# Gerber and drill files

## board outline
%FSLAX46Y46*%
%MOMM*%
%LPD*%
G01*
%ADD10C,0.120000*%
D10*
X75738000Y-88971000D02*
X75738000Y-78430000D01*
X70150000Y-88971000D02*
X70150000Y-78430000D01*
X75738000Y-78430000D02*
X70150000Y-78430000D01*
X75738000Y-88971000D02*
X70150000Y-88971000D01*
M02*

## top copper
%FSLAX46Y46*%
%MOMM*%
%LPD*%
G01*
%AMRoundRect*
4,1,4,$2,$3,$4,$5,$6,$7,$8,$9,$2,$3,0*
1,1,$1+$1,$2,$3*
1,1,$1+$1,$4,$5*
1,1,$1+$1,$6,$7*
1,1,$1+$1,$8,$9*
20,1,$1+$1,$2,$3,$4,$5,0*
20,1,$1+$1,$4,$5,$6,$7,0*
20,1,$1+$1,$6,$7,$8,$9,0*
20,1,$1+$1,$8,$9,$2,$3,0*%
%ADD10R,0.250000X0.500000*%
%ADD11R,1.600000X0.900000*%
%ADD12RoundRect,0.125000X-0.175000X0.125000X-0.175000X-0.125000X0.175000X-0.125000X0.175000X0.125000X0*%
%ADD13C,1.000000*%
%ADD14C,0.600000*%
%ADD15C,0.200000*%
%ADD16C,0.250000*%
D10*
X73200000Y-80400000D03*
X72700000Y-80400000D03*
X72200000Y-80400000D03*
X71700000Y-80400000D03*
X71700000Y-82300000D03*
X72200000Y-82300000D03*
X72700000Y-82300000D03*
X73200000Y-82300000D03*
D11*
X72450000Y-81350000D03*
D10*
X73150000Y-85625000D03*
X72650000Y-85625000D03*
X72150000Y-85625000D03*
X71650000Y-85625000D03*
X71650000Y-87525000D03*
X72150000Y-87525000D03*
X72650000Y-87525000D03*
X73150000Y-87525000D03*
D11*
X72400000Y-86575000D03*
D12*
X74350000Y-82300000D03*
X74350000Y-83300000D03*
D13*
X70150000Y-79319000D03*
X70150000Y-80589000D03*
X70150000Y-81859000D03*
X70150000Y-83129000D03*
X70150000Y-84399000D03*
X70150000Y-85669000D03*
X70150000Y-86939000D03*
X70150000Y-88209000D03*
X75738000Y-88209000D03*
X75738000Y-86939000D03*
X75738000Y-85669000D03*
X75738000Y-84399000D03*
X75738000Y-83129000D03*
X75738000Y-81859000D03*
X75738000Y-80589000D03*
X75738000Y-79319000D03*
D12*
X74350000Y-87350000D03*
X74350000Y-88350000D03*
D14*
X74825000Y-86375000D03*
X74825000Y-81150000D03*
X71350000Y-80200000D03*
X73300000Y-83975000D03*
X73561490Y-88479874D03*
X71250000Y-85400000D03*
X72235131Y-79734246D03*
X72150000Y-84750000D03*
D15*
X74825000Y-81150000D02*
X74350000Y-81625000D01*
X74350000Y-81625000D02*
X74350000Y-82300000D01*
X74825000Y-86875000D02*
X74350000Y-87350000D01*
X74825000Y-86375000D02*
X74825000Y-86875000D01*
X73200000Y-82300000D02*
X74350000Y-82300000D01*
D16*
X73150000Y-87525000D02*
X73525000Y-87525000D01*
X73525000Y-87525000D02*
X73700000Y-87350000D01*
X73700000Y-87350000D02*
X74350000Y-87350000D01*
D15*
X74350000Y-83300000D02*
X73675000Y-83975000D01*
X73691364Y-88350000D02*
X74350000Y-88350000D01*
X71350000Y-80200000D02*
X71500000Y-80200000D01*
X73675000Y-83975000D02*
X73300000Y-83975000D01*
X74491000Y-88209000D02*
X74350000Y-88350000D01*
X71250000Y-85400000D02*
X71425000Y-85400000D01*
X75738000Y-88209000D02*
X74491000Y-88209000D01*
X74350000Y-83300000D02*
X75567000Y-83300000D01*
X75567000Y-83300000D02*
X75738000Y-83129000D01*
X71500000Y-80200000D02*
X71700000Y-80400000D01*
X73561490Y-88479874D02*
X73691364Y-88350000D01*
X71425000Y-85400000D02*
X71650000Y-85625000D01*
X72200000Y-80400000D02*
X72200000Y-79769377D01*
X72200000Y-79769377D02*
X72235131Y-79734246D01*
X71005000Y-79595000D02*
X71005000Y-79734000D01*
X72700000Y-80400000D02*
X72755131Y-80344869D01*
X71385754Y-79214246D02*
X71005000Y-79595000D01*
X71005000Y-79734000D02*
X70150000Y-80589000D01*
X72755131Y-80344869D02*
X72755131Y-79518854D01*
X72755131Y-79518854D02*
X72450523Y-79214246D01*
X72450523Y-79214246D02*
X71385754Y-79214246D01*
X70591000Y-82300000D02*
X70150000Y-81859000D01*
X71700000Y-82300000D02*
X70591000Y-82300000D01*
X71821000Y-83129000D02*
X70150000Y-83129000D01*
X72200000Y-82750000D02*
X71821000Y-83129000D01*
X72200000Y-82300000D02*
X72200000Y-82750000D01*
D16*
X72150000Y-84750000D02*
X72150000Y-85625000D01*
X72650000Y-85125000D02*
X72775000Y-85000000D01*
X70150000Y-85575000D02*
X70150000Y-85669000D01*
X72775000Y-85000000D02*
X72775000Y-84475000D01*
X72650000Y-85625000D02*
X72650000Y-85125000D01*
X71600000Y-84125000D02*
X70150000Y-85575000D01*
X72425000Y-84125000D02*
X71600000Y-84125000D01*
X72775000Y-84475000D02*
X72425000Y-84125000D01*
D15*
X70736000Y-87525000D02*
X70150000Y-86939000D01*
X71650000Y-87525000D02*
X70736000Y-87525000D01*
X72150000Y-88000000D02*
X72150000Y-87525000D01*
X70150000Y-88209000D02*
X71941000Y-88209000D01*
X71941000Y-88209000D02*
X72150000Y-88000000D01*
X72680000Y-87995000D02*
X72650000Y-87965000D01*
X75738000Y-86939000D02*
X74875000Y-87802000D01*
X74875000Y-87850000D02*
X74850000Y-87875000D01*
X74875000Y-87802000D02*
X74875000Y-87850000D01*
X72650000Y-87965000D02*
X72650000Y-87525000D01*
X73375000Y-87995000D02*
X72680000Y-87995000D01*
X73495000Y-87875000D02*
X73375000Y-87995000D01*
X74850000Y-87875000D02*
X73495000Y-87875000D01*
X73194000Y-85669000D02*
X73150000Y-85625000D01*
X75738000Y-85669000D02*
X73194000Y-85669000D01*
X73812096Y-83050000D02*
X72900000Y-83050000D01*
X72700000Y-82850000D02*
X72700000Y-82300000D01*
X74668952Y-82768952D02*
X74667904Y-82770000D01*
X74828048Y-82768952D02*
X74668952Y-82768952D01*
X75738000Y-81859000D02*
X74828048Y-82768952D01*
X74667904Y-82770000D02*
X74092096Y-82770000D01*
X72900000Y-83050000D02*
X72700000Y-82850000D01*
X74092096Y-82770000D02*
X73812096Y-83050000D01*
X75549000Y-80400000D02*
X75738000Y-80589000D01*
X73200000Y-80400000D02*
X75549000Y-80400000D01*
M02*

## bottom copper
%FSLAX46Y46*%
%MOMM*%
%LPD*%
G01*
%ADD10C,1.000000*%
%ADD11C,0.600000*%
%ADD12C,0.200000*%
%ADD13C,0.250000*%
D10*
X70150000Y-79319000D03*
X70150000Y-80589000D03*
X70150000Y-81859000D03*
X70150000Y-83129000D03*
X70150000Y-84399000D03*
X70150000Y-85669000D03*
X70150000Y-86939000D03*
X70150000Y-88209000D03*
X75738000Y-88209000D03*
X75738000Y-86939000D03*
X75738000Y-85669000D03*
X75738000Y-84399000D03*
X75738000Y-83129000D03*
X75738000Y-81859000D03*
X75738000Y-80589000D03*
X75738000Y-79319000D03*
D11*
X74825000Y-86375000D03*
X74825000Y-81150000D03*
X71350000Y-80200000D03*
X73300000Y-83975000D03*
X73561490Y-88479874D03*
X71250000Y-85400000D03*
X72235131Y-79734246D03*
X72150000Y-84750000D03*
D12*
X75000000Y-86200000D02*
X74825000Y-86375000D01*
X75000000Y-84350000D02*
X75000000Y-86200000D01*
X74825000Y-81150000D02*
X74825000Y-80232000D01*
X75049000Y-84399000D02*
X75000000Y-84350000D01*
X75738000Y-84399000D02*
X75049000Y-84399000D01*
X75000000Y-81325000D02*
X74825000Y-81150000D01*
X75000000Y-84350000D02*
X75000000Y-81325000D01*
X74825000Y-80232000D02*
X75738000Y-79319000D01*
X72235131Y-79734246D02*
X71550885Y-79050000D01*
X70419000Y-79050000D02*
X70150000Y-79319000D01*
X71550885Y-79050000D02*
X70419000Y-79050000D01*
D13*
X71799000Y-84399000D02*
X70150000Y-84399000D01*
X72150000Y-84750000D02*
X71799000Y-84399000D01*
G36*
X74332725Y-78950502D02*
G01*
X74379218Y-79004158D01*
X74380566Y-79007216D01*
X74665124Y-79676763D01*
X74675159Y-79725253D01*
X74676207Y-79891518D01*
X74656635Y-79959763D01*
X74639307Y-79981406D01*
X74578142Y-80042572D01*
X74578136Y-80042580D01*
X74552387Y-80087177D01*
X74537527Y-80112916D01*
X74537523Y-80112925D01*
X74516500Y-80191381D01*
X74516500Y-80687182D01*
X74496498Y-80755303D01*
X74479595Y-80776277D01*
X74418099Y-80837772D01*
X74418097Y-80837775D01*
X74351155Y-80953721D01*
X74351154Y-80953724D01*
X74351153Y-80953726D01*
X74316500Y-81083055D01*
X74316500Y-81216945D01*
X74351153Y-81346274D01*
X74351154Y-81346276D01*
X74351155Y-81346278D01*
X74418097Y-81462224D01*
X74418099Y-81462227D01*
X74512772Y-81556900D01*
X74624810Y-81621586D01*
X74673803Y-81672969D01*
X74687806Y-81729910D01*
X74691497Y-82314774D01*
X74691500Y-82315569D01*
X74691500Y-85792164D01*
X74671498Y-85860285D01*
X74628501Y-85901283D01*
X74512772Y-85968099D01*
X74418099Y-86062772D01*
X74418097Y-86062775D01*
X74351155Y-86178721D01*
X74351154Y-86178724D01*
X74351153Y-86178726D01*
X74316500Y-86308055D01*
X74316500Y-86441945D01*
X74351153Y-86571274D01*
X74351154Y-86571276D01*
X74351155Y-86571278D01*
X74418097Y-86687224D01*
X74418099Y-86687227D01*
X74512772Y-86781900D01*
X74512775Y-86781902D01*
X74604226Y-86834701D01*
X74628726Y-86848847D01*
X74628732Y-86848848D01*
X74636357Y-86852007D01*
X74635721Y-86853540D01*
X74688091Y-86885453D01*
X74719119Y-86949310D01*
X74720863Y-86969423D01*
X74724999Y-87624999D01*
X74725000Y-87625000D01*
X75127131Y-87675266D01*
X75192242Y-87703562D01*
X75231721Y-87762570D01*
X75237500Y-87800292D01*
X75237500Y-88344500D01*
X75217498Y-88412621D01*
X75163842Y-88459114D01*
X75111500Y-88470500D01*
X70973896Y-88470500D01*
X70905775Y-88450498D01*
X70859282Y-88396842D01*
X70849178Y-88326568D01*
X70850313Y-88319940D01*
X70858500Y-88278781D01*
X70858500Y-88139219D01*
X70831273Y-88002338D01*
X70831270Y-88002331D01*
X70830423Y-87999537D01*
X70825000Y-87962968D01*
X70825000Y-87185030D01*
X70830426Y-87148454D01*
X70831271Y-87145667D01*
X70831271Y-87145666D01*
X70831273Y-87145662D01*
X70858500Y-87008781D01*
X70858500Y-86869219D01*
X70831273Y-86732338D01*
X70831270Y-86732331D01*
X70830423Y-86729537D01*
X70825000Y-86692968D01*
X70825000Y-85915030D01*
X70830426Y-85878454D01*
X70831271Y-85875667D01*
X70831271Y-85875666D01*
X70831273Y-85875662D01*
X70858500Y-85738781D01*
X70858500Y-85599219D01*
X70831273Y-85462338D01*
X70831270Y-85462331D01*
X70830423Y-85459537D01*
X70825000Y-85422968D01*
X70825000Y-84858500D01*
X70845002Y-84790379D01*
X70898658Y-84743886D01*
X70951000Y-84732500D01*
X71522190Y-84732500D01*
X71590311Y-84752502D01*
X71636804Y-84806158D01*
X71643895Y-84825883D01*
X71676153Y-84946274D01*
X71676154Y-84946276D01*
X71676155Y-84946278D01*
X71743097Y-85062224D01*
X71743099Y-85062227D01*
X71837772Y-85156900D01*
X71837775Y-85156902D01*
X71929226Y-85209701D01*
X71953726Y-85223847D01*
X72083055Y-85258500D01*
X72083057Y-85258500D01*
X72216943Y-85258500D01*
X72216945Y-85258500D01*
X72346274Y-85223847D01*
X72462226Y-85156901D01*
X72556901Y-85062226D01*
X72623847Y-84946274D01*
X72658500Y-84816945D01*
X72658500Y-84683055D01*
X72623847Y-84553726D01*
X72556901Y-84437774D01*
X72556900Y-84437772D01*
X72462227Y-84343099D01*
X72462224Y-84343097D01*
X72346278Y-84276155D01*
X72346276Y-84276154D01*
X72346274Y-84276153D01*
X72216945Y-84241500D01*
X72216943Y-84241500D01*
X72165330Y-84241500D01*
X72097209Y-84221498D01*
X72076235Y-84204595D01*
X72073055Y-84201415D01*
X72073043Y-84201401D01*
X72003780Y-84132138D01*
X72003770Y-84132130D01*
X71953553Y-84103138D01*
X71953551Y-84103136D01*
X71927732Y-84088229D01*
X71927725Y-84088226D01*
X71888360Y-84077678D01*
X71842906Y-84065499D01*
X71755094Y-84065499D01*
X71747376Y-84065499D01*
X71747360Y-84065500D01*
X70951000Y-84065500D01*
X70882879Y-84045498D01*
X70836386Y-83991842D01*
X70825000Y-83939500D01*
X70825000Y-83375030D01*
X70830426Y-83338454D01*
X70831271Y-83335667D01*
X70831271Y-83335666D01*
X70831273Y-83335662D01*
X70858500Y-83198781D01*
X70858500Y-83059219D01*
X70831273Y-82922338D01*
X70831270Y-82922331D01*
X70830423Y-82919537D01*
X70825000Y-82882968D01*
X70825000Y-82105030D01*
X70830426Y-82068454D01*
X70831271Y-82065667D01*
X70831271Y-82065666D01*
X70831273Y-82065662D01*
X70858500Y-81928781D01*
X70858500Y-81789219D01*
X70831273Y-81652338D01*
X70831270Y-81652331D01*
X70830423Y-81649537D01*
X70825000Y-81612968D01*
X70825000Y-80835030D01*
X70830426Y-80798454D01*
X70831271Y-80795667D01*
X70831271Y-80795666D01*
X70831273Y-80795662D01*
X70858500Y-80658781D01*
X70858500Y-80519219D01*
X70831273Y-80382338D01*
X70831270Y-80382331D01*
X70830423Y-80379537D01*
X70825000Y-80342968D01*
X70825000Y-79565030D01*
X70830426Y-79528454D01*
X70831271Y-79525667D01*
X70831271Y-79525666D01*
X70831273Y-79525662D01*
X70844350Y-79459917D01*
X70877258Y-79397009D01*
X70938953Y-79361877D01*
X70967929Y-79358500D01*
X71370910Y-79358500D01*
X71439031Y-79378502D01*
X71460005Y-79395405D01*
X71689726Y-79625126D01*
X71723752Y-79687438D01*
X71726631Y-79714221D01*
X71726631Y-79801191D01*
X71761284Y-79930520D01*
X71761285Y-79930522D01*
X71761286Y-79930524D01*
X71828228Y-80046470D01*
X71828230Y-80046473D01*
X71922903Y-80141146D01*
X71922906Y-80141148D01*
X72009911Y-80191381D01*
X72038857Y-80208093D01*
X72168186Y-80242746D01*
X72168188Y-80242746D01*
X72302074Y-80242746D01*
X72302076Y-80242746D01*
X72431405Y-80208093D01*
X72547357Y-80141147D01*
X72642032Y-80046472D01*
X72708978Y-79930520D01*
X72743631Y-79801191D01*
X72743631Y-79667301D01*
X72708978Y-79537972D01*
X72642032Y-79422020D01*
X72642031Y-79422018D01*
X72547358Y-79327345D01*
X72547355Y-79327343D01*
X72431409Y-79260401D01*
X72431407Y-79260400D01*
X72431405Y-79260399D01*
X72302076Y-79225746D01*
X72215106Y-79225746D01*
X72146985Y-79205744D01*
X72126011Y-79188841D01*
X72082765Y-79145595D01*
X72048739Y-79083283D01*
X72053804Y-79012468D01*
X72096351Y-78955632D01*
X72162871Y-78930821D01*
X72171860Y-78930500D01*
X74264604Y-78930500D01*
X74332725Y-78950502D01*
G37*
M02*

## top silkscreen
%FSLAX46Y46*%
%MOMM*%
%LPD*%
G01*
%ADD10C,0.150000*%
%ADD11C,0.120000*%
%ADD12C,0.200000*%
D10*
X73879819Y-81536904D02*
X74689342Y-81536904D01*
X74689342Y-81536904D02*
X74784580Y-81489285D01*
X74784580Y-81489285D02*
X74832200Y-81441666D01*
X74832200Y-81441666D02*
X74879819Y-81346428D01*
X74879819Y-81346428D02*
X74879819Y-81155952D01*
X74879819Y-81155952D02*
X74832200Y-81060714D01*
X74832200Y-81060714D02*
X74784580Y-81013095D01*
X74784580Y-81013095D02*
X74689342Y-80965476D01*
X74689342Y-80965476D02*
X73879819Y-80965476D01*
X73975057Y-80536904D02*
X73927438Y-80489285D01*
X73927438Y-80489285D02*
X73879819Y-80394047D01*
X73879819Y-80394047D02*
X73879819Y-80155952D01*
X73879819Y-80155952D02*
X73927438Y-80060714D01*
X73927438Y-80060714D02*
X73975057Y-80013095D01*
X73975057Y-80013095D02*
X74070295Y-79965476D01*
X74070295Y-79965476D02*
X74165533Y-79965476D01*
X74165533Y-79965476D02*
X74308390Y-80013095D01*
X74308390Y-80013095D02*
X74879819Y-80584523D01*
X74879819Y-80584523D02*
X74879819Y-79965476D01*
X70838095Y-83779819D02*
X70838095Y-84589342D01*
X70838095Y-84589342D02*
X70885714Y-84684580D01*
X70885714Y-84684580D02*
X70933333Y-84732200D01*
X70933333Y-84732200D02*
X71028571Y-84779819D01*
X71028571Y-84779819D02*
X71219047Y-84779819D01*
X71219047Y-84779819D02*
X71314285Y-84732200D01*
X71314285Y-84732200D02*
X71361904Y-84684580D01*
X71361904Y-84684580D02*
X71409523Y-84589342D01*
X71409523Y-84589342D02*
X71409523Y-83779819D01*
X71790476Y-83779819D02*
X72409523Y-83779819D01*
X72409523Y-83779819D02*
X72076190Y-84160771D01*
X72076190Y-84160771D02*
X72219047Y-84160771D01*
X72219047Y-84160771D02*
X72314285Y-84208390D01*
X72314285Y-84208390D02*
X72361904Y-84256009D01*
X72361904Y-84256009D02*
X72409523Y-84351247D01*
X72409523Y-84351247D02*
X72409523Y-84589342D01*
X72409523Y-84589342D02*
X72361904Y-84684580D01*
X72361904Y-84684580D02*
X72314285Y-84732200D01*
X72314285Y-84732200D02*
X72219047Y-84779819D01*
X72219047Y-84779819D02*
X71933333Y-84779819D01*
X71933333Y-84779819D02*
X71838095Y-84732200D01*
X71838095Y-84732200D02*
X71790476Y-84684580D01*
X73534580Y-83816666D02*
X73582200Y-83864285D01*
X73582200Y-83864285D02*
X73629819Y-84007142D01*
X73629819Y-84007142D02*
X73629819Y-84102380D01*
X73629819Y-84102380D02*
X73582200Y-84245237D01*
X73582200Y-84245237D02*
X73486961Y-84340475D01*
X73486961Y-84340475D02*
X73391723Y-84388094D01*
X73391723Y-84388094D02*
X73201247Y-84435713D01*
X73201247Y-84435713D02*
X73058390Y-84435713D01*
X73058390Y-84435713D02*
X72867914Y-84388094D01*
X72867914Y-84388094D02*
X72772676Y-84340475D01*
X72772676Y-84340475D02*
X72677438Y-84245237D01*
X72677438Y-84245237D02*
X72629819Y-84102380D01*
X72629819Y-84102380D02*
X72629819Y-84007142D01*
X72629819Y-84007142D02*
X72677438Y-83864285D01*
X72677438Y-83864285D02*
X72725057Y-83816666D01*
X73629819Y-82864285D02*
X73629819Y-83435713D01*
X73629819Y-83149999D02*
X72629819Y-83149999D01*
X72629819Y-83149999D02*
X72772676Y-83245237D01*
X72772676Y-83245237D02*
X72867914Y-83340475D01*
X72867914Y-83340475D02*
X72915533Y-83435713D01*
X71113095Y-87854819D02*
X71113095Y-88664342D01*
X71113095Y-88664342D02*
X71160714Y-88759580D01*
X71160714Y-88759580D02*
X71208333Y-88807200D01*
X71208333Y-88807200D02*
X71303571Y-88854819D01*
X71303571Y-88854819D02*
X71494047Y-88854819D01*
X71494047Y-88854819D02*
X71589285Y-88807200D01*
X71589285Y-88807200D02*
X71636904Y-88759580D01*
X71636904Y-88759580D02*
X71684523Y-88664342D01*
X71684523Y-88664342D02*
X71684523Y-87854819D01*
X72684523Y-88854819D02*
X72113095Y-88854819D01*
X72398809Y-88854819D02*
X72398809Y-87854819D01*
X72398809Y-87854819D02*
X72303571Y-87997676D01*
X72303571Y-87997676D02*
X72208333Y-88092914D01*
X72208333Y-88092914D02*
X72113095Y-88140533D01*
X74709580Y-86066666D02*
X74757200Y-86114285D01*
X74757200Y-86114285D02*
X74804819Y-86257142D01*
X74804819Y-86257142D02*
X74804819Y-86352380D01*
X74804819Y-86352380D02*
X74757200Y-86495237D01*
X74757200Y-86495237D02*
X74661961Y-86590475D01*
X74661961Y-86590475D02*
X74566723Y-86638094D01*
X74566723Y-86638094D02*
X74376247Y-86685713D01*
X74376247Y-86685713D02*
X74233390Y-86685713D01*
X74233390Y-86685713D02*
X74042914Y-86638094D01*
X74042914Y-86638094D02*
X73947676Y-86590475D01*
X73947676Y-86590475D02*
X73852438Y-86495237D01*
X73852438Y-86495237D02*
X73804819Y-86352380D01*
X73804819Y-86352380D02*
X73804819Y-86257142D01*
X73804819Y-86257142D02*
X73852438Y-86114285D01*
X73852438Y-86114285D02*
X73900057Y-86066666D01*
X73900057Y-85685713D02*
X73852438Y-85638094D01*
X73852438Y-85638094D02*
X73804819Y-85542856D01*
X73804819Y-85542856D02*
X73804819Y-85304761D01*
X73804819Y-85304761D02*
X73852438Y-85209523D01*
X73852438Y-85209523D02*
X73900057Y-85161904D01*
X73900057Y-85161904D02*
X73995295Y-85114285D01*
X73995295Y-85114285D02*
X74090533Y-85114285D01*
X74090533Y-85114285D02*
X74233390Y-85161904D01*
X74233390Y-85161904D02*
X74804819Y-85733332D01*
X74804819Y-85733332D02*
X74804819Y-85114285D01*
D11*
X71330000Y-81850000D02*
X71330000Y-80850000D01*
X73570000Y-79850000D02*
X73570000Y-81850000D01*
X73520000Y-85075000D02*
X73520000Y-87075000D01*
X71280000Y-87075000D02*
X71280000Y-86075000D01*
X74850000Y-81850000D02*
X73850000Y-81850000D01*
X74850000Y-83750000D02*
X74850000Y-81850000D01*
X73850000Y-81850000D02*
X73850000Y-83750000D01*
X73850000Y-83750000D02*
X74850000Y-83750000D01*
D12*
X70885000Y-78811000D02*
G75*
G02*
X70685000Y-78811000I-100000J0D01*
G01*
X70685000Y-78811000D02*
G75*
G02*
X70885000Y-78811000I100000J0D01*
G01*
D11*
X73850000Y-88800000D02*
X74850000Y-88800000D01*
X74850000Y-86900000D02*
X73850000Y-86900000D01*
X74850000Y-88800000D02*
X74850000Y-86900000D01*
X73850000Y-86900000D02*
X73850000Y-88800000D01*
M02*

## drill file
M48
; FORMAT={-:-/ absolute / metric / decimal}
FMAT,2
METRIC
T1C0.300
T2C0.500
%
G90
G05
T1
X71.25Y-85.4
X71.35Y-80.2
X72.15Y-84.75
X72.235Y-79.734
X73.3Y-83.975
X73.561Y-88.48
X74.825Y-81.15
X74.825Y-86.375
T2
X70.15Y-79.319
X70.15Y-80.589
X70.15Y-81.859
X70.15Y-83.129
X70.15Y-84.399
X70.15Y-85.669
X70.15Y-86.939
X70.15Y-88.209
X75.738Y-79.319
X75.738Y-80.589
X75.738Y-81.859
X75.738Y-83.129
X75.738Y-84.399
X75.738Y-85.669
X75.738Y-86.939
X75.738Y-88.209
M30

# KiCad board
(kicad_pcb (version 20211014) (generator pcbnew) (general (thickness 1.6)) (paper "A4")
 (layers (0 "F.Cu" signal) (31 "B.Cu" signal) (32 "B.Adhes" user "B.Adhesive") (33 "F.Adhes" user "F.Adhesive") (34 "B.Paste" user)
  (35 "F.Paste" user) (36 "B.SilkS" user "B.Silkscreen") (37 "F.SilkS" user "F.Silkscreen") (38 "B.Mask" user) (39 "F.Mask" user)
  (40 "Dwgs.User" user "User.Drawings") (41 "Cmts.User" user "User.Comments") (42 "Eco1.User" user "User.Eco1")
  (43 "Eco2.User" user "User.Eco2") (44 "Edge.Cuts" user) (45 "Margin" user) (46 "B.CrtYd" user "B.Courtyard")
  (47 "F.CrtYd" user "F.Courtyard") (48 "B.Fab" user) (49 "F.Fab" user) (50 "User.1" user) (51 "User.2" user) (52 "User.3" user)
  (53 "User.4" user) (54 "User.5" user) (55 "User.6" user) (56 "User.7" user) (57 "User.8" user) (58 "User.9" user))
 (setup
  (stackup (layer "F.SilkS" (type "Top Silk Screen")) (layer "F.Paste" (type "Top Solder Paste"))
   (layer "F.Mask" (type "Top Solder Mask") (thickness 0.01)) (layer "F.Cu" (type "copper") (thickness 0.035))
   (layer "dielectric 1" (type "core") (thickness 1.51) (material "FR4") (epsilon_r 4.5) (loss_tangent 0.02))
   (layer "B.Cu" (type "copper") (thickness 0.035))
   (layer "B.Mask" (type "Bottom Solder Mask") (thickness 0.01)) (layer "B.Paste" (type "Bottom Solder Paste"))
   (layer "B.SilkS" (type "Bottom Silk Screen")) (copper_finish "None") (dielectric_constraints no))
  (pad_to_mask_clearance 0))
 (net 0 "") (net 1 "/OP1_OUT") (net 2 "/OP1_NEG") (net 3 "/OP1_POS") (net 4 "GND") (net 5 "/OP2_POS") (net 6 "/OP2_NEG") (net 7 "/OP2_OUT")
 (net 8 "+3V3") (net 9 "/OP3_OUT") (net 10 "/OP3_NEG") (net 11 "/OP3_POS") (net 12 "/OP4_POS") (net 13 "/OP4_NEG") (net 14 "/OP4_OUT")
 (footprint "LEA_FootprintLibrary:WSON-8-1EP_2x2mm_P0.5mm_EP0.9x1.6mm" (layer "F.Cu") (at 72.45 81.35 -90)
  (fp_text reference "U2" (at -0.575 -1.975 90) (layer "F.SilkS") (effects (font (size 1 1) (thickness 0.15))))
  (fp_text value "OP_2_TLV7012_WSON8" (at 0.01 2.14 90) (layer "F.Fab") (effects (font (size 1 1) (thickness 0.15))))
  (fp_line (start 0.5 1.12) (end -0.5 1.12) (layer "F.SilkS") (width 0.12))
  (fp_line (start -1.5 -1.12) (end 0.5 -1.12) (layer "F.SilkS") (width 0.12))
  (pad "" smd rect (at 0 -0.4 270) (size 0.75 0.65) (layers "F.Paste"))
  (pad "" smd rect (at 0 0.4 270) (size 0.75 0.65) (layers "F.Paste"))
  (pad "1" smd rect (at -0.95 -0.75 270) (size 0.5 0.25) (layers "F.Cu" "F.Paste" "F.Mask") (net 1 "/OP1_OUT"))
  (pad "2" smd rect (at -0.95 -0.25 270) (size 0.5 0.25) (layers "F.Cu" "F.Paste" "F.Mask") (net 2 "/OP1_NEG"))
  (pad "3" smd rect (at -0.95 0.25 270) (size 0.5 0.25) (layers "F.Cu" "F.Paste" "F.Mask") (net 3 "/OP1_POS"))
  (pad "4" smd rect (at -0.95 0.75 270) (size 0.5 0.25) (layers "F.Cu" "F.Paste" "F.Mask") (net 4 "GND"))
  (pad "5" smd rect (at 0.95 0.75 270) (size 0.5 0.25) (layers "F.Cu" "F.Paste" "F.Mask") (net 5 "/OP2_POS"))
  (pad "6" smd rect (at 0.95 0.25 270) (size 0.5 0.25) (layers "F.Cu" "F.Paste" "F.Mask") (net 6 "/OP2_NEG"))
  (pad "7" smd rect (at 0.95 -0.25 270) (size 0.5 0.25) (layers "F.Cu" "F.Paste" "F.Mask") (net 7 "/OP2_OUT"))
  (pad "8" smd rect (at 0.95 -0.75 270) (size 0.5 0.25) (layers "F.Cu" "F.Paste" "F.Mask") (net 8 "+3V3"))
  (pad "9" smd rect (at 0 0 270) (size 0.9 1.6) (layers "F.Cu" "F.Mask")))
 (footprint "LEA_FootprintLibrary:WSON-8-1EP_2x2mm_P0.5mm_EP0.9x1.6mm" (layer "F.Cu") (at 72.4 86.575 -90)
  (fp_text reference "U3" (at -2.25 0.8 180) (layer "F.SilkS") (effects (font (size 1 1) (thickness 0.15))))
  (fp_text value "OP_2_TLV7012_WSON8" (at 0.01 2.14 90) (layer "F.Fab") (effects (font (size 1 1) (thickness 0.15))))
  (fp_line (start -1.5 -1.12) (end 0.5 -1.12) (layer "F.SilkS") (width 0.12))
  (fp_line (start 0.5 1.12) (end -0.5 1.12) (layer "F.SilkS") (width 0.12))
  (pad "" smd rect (at 0 -0.4 270) (size 0.75 0.65) (layers "F.Paste"))
  (pad "" smd rect (at 0 0.4 270) (size 0.75 0.65) (layers "F.Paste"))
  (pad "1" smd rect (at -0.95 -0.75 270) (size 0.5 0.25) (layers "F.Cu" "F.Paste" "F.Mask") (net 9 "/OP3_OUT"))
  (pad "2" smd rect (at -0.95 -0.25 270) (size 0.5 0.25) (layers "F.Cu" "F.Paste" "F.Mask") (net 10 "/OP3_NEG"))
  (pad "3" smd rect (at -0.95 0.25 270) (size 0.5 0.25) (layers "F.Cu" "F.Paste" "F.Mask") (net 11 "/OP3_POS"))
  (pad "4" smd rect (at -0.95 0.75 270) (size 0.5 0.25) (layers "F.Cu" "F.Paste" "F.Mask") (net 4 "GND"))
  (pad "5" smd rect (at 0.95 0.75 270) (size 0.5 0.25) (layers "F.Cu" "F.Paste" "F.Mask") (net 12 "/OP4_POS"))
  (pad "6" smd rect (at 0.95 0.25 270) (size 0.5 0.25) (layers "F.Cu" "F.Paste" "F.Mask") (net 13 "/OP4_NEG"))
  (pad "7" smd rect (at 0.95 -0.25 270) (size 0.5 0.25) (layers "F.Cu" "F.Paste" "F.Mask") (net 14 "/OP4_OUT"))
  (pad "8" smd rect (at 0.95 -0.75 270) (size 0.5 0.25) (layers "F.Cu" "F.Paste" "F.Mask") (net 8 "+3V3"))
  (pad "9" smd rect (at 0 0 270) (size 0.9 1.6) (layers "F.Cu" "F.Mask")))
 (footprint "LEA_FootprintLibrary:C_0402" (layer "F.Cu") (at 74.35 82.8 -90)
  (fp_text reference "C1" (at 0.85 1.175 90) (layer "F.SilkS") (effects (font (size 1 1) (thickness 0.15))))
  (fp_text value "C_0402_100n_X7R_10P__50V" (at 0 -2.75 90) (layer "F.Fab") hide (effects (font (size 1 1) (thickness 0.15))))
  (fp_line (start -0.95 -0.5) (end -0.95 0.5) (layer "F.SilkS") (width 0.12))
  (fp_line (start 0.95 -0.5) (end -0.95 -0.5) (layer "F.SilkS") (width 0.12))
  (fp_line (start -0.95 0.5) (end 0.95 0.5) (layer "F.SilkS") (width 0.12))
  (fp_line (start 0.95 0.5) (end 0.95 -0.5) (layer "F.SilkS") (width 0.12))
  (pad "1" smd roundrect (at -0.5 0 270) (size 0.5 0.6) (layers "F.Cu" "F.Paste" "F.Mask") (roundrect_rratio 0.25) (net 8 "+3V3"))
  (pad "2" smd roundrect (at 0.5 0 270) (size 0.5 0.6) (layers "F.Cu" "F.Paste" "F.Mask") (roundrect_rratio 0.25) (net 4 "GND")))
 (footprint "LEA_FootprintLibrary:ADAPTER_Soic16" (layer "F.Cu") (at 73.325 83.764)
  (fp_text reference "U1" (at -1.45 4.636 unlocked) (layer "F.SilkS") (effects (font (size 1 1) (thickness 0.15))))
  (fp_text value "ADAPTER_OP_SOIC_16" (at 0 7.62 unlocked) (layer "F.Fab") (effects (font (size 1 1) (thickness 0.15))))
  (fp_circle (center -2.54 -4.953) (end -2.54 -4.853) (layer "F.SilkS") (width 0.2) (fill none))
  (fp_line (start 2.413 5.207) (end 2.413 -5.334) (layer "Edge.Cuts") (width 0.12))
  (fp_line (start -3.175 5.207) (end -3.175 -5.334) (layer "Edge.Cuts") (width 0.12))
  (fp_line (start 2.413 -5.334) (end -3.175 -5.334) (layer "Edge.Cuts") (width 0.12))
  (fp_line (start 2.413 5.207) (end -3.175 5.207) (layer "Edge.Cuts") (width 0.12))
  (pad "1" thru_hole circle (at -3.175 -4.445) (size 1 1) (drill 0.5) (layers *.Cu *.Mask) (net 3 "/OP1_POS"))
  (pad "2" thru_hole circle (at -3.175 -3.175) (size 1 1) (drill 0.5) (layers *.Cu *.Mask) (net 2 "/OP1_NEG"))
  (pad "3" thru_hole circle (at -3.175 -1.905) (size 1 1) (drill 0.5) (layers *.Cu *.Mask) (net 5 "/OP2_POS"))
  (pad "4" thru_hole circle (at -3.175 -0.635) (size 1 1) (drill 0.5) (layers *.Cu *.Mask) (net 6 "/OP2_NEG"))
  (pad "5" thru_hole circle (at -3.175 0.635) (size 1 1) (drill 0.5) (layers *.Cu *.Mask) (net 11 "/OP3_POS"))
  (pad "6" thru_hole circle (at -3.175 1.905) (size 1 1) (drill 0.5) (layers *.Cu *.Mask) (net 10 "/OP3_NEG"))
  (pad "7" thru_hole circle (at -3.175 3.175) (size 1 1) (drill 0.5) (layers *.Cu *.Mask) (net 12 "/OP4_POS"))
  (pad "8" thru_hole circle (at -3.175 4.445) (size 1 1) (drill 0.5) (layers *.Cu *.Mask) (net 13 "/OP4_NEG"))
  (pad "9" thru_hole circle (at 2.413 4.445) (size 1 1) (drill 0.5) (layers *.Cu *.Mask) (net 4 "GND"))
  (pad "10" thru_hole circle (at 2.413 3.175) (size 1 1) (drill 0.5) (layers *.Cu *.Mask) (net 14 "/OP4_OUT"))
  (pad "11" thru_hole circle (at 2.413 1.905) (size 1 1) (drill 0.5) (layers *.Cu *.Mask) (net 9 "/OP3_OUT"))
  (pad "12" thru_hole circle (at 2.413 0.635) (size 1 1) (drill 0.5) (layers *.Cu *.Mask) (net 8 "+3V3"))
  (pad "13" thru_hole circle (at 2.413 -0.635) (size 1 1) (drill 0.5) (layers *.Cu *.Mask) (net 4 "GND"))
  (pad "14" thru_hole circle (at 2.413 -1.905) (size 1 1) (drill 0.5) (layers *.Cu *.Mask) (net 7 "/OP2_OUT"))
  (pad "15" thru_hole circle (at 2.413 -3.175) (size 1 1) (drill 0.5) (layers *.Cu *.Mask) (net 1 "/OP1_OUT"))
  (pad "16" thru_hole circle (at 2.413 -4.445) (size 1 1) (drill 0.5) (layers *.Cu *.Mask) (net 8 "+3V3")))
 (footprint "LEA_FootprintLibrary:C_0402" (layer "F.Cu") (at 74.35 87.85 -90)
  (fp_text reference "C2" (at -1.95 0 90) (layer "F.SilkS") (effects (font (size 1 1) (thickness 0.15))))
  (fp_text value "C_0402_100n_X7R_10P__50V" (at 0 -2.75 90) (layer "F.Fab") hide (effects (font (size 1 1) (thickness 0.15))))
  (fp_line (start 0.95 0.5) (end 0.95 -0.5) (layer "F.SilkS") (width 0.12))
  (fp_line (start -0.95 -0.5) (end -0.95 0.5) (layer "F.SilkS") (width 0.12))
  (fp_line (start 0.95 -0.5) (end -0.95 -0.5) (layer "F.SilkS") (width 0.12))
  (fp_line (start -0.95 0.5) (end 0.95 0.5) (layer "F.SilkS") (width 0.12))
  (pad "1" smd roundrect (at -0.5 0 270) (size 0.5 0.6) (layers "F.Cu" "F.Paste" "F.Mask") (roundrect_rratio 0.25) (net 8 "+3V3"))
  (pad "2" smd roundrect (at 0.5 0 270) (size 0.5 0.6) (layers "F.Cu" "F.Paste" "F.Mask") (roundrect_rratio 0.25) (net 4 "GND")))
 (segment (start 74.825 81.15) (end 74.35 81.625) (width 0.2) (layer "F.Cu") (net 8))
 (segment (start 74.35 81.625) (end 74.35 82.3) (width 0.2) (layer "F.Cu") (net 8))
 (segment (start 74.825 86.875) (end 74.35 87.35) (width 0.2) (layer "F.Cu") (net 8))
 (segment (start 74.825 86.375) (end 74.825 86.875) (width 0.2) (layer "F.Cu") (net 8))
 (segment (start 73.2 82.3) (end 74.35 82.3) (width 0.2) (layer "F.Cu") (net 8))
 (segment (start 73.15 87.525) (end 73.525 87.525) (width 0.25) (layer "F.Cu") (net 8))
 (segment (start 73.525 87.525) (end 73.7 87.35) (width 0.25) (layer "F.Cu") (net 8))
 (segment (start 73.7 87.35) (end 74.35 87.35) (width 0.25) (layer "F.Cu") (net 8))
 (via (at 74.825 86.375) (size 0.6) (drill 0.3) (layers "F.Cu" "B.Cu") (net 8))
 (via (at 74.825 81.15) (size 0.6) (drill 0.3) (layers "F.Cu" "B.Cu") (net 8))
 (segment (start 75 86.2) (end 74.825 86.375) (width 0.2) (layer "B.Cu") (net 8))
 (segment (start 75 84.35) (end 75 86.2) (width 0.2) (layer "B.Cu") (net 8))
 (segment (start 74.825 81.15) (end 74.825 80.232) (width 0.2) (layer "B.Cu") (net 8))
 (segment (start 75.049 84.399) (end 75 84.35) (width 0.2) (layer "B.Cu") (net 8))
 (segment (start 75.738 84.399) (end 75.049 84.399) (width 0.2) (layer "B.Cu") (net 8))
 (segment (start 75 81.325) (end 74.825 81.15) (width 0.2) (layer "B.Cu") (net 8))
 (segment (start 75 84.35) (end 75 81.325) (width 0.2) (layer "B.Cu") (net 8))
 (segment (start 74.825 80.232) (end 75.738 79.319) (width 0.2) (layer "B.Cu") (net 8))
 (segment (start 74.35 83.3) (end 73.675 83.975) (width 0.2) (layer "F.Cu") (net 4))
 (segment (start 73.691364 88.35) (end 74.35 88.35) (width 0.2) (layer "F.Cu") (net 4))
 (segment (start 71.35 80.2) (end 71.5 80.2) (width 0.2) (layer "F.Cu") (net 4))
 (segment (start 73.675 83.975) (end 73.3 83.975) (width 0.2) (layer "F.Cu") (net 4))
 (segment (start 74.491 88.209) (end 74.35 88.35) (width 0.2) (layer "F.Cu") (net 4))
 (segment (start 71.25 85.4) (end 71.425 85.4) (width 0.2) (layer "F.Cu") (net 4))
 (segment (start 75.738 88.209) (end 74.491 88.209) (width 0.2) (layer "F.Cu") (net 4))
 (segment (start 74.35 83.3) (end 75.567 83.3) (width 0.2) (layer "F.Cu") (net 4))
 (segment (start 75.567 83.3) (end 75.738 83.129) (width 0.2) (layer "F.Cu") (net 4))
 (segment (start 71.5 80.2) (end 71.7 80.4) (width 0.2) (layer "F.Cu") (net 4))
 (segment (start 73.56149 88.479874) (end 73.691364 88.35) (width 0.2) (layer "F.Cu") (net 4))
 (segment (start 71.425 85.4) (end 71.65 85.625) (width 0.2) (layer "F.Cu") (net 4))
 (via (at 71.35 80.2) (size 0.6) (drill 0.3) (layers "F.Cu" "B.Cu") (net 4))
 (via (at 73.3 83.975) (size 0.6) (drill 0.3) (layers "F.Cu" "B.Cu") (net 4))
 (via (at 73.56149 88.479874) (size 0.6) (drill 0.3) (layers "F.Cu" "B.Cu") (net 4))
 (via (at 71.25 85.4) (size 0.6) (drill 0.3) (layers "F.Cu" "B.Cu") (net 4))
 (segment (start 72.2 80.4) (end 72.2 79.769377) (width 0.2) (layer "F.Cu") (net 3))
 (segment (start 72.2 79.769377) (end 72.235131 79.734246) (width 0.2) (layer "F.Cu") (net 3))
 (via (at 72.235131 79.734246) (size 0.6) (drill 0.3) (layers "F.Cu" "B.Cu") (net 3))
 (segment (start 72.235131 79.734246) (end 71.550885 79.05) (width 0.2) (layer "B.Cu") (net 3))
 (segment (start 70.419 79.05) (end 70.15 79.319) (width 0.2) (layer "B.Cu") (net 3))
 (segment (start 71.550885 79.05) (end 70.419 79.05) (width 0.2) (layer "B.Cu") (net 3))
 (segment (start 71.005 79.595) (end 71.005 79.734) (width 0.2) (layer "F.Cu") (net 2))
 (segment (start 72.7 80.4) (end 72.755131 80.344869) (width 0.2) (layer "F.Cu") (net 2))
 (segment (start 71.385754 79.214246) (end 71.005 79.595) (width 0.2) (layer "F.Cu") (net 2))
 (segment (start 71.005 79.734) (end 70.15 80.589) (width 0.2) (layer "F.Cu") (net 2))
 (segment (start 72.755131 80.344869) (end 72.755131 79.518854) (width 0.2) (layer "F.Cu") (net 2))
 (segment (start 72.755131 79.518854) (end 72.450523 79.214246) (width 0.2) (layer "F.Cu") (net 2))
 (segment (start 72.450523 79.214246) (end 71.385754 79.214246) (width 0.2) (layer "F.Cu") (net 2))
 (segment (start 70.591 82.3) (end 70.15 81.859) (width 0.2) (layer "F.Cu") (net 5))
 (segment (start 71.7 82.3) (end 70.591 82.3) (width 0.2) (layer "F.Cu") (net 5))
 (segment (start 71.821 83.129) (end 70.15 83.129) (width 0.2) (layer "F.Cu") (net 6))
 (segment (start 72.2 82.75) (end 71.821 83.129) (width 0.2) (layer "F.Cu") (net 6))
 (segment (start 72.2 82.3) (end 72.2 82.75) (width 0.2) (layer "F.Cu") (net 6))
 (segment (start 72.15 84.75) (end 72.15 85.625) (width 0.25) (layer "F.Cu") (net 11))
 (via (at 72.15 84.75) (size 0.6) (drill 0.3) (layers "F.Cu" "B.Cu") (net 11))
 (segment (start 71.799 84.399) (end 70.15 84.399) (width 0.25) (layer "B.Cu") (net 11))
 (segment (start 72.15 84.75) (end 71.799 84.399) (width 0.25) (layer "B.Cu") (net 11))
 (segment (start 72.65 85.125) (end 72.775 85) (width 0.25) (layer "F.Cu") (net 10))
 (segment (start 70.15 85.575) (end 70.15 85.669) (width 0.25) (layer "F.Cu") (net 10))
 (segment (start 72.775 85) (end 72.775 84.475) (width 0.25) (layer "F.Cu") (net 10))
 (segment (start 72.65 85.625) (end 72.65 85.125) (width 0.25) (layer "F.Cu") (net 10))
 (segment (start 71.6 84.125) (end 70.15 85.575) (width 0.25) (layer "F.Cu") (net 10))
 (segment (start 72.425 84.125) (end 71.6 84.125) (width 0.25) (layer "F.Cu") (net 10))
 (segment (start 72.775 84.475) (end 72.425 84.125) (width 0.25) (layer "F.Cu") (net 10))
 (segment (start 70.736 87.525) (end 70.15 86.939) (width 0.2) (layer "F.Cu") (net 12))
 (segment (start 71.65 87.525) (end 70.736 87.525) (width 0.2) (layer "F.Cu") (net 12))
 (segment (start 72.15 88) (end 72.15 87.525) (width 0.2) (layer "F.Cu") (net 13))
 (segment (start 70.15 88.209) (end 71.941 88.209) (width 0.2) (layer "F.Cu") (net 13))
 (segment (start 71.941 88.209) (end 72.15 88) (width 0.2) (layer "F.Cu") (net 13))
 (segment (start 72.68 87.995) (end 72.65 87.965) (width 0.2) (layer "F.Cu") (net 14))
 (segment (start 75.738 86.939) (end 74.875 87.802) (width 0.2) (layer "F.Cu") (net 14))
 (segment (start 74.875 87.85) (end 74.85 87.875) (width 0.2) (layer "F.Cu") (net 14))
 (segment (start 74.875 87.802) (end 74.875 87.85) (width 0.2) (layer "F.Cu") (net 14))
 (segment (start 72.65 87.965) (end 72.65 87.525) (width 0.2) (layer "F.Cu") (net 14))
 (segment (start 73.375 87.995) (end 72.68 87.995) (width 0.2) (layer "F.Cu") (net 14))
 (segment (start 73.495 87.875) (end 73.375 87.995) (width 0.2) (layer "F.Cu") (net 14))
 (segment (start 74.85 87.875) (end 73.495 87.875) (width 0.2) (layer "F.Cu") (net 14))
 (segment (start 73.194 85.669) (end 73.15 85.625) (width 0.2) (layer "F.Cu") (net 9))
 (segment (start 75.738 85.669) (end 73.194 85.669) (width 0.2) (layer "F.Cu") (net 9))
 (segment (start 73.812096 83.05) (end 72.9 83.05) (width 0.2) (layer "F.Cu") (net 7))
 (segment (start 72.7 82.85) (end 72.7 82.3) (width 0.2) (layer "F.Cu") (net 7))
 (segment (start 74.668952 82.768952) (end 74.667904 82.77) (width 0.2) (layer "F.Cu") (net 7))
 (segment (start 74.828048 82.768952) (end 74.668952 82.768952) (width 0.2) (layer "F.Cu") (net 7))
 (segment (start 75.738 81.859) (end 74.828048 82.768952) (width 0.2) (layer "F.Cu") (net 7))
 (segment (start 74.667904 82.77) (end 74.092096 82.77) (width 0.2) (layer "F.Cu") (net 7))
 (segment (start 72.9 83.05) (end 72.7 82.85) (width 0.2) (layer "F.Cu") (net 7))
 (segment (start 74.092096 82.77) (end 73.812096 83.05) (width 0.2) (layer "F.Cu") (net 7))
 (segment (start 75.549 80.4) (end 75.738 80.589) (width 0.2) (layer "F.Cu") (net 1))
 (segment (start 73.2 80.4) (end 75.549 80.4) (width 0.2) (layer "F.Cu") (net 1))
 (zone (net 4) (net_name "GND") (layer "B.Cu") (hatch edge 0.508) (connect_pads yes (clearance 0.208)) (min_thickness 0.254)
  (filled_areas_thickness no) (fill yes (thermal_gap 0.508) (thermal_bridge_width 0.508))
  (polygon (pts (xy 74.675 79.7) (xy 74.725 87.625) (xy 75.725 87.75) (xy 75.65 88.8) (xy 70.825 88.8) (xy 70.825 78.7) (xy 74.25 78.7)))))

